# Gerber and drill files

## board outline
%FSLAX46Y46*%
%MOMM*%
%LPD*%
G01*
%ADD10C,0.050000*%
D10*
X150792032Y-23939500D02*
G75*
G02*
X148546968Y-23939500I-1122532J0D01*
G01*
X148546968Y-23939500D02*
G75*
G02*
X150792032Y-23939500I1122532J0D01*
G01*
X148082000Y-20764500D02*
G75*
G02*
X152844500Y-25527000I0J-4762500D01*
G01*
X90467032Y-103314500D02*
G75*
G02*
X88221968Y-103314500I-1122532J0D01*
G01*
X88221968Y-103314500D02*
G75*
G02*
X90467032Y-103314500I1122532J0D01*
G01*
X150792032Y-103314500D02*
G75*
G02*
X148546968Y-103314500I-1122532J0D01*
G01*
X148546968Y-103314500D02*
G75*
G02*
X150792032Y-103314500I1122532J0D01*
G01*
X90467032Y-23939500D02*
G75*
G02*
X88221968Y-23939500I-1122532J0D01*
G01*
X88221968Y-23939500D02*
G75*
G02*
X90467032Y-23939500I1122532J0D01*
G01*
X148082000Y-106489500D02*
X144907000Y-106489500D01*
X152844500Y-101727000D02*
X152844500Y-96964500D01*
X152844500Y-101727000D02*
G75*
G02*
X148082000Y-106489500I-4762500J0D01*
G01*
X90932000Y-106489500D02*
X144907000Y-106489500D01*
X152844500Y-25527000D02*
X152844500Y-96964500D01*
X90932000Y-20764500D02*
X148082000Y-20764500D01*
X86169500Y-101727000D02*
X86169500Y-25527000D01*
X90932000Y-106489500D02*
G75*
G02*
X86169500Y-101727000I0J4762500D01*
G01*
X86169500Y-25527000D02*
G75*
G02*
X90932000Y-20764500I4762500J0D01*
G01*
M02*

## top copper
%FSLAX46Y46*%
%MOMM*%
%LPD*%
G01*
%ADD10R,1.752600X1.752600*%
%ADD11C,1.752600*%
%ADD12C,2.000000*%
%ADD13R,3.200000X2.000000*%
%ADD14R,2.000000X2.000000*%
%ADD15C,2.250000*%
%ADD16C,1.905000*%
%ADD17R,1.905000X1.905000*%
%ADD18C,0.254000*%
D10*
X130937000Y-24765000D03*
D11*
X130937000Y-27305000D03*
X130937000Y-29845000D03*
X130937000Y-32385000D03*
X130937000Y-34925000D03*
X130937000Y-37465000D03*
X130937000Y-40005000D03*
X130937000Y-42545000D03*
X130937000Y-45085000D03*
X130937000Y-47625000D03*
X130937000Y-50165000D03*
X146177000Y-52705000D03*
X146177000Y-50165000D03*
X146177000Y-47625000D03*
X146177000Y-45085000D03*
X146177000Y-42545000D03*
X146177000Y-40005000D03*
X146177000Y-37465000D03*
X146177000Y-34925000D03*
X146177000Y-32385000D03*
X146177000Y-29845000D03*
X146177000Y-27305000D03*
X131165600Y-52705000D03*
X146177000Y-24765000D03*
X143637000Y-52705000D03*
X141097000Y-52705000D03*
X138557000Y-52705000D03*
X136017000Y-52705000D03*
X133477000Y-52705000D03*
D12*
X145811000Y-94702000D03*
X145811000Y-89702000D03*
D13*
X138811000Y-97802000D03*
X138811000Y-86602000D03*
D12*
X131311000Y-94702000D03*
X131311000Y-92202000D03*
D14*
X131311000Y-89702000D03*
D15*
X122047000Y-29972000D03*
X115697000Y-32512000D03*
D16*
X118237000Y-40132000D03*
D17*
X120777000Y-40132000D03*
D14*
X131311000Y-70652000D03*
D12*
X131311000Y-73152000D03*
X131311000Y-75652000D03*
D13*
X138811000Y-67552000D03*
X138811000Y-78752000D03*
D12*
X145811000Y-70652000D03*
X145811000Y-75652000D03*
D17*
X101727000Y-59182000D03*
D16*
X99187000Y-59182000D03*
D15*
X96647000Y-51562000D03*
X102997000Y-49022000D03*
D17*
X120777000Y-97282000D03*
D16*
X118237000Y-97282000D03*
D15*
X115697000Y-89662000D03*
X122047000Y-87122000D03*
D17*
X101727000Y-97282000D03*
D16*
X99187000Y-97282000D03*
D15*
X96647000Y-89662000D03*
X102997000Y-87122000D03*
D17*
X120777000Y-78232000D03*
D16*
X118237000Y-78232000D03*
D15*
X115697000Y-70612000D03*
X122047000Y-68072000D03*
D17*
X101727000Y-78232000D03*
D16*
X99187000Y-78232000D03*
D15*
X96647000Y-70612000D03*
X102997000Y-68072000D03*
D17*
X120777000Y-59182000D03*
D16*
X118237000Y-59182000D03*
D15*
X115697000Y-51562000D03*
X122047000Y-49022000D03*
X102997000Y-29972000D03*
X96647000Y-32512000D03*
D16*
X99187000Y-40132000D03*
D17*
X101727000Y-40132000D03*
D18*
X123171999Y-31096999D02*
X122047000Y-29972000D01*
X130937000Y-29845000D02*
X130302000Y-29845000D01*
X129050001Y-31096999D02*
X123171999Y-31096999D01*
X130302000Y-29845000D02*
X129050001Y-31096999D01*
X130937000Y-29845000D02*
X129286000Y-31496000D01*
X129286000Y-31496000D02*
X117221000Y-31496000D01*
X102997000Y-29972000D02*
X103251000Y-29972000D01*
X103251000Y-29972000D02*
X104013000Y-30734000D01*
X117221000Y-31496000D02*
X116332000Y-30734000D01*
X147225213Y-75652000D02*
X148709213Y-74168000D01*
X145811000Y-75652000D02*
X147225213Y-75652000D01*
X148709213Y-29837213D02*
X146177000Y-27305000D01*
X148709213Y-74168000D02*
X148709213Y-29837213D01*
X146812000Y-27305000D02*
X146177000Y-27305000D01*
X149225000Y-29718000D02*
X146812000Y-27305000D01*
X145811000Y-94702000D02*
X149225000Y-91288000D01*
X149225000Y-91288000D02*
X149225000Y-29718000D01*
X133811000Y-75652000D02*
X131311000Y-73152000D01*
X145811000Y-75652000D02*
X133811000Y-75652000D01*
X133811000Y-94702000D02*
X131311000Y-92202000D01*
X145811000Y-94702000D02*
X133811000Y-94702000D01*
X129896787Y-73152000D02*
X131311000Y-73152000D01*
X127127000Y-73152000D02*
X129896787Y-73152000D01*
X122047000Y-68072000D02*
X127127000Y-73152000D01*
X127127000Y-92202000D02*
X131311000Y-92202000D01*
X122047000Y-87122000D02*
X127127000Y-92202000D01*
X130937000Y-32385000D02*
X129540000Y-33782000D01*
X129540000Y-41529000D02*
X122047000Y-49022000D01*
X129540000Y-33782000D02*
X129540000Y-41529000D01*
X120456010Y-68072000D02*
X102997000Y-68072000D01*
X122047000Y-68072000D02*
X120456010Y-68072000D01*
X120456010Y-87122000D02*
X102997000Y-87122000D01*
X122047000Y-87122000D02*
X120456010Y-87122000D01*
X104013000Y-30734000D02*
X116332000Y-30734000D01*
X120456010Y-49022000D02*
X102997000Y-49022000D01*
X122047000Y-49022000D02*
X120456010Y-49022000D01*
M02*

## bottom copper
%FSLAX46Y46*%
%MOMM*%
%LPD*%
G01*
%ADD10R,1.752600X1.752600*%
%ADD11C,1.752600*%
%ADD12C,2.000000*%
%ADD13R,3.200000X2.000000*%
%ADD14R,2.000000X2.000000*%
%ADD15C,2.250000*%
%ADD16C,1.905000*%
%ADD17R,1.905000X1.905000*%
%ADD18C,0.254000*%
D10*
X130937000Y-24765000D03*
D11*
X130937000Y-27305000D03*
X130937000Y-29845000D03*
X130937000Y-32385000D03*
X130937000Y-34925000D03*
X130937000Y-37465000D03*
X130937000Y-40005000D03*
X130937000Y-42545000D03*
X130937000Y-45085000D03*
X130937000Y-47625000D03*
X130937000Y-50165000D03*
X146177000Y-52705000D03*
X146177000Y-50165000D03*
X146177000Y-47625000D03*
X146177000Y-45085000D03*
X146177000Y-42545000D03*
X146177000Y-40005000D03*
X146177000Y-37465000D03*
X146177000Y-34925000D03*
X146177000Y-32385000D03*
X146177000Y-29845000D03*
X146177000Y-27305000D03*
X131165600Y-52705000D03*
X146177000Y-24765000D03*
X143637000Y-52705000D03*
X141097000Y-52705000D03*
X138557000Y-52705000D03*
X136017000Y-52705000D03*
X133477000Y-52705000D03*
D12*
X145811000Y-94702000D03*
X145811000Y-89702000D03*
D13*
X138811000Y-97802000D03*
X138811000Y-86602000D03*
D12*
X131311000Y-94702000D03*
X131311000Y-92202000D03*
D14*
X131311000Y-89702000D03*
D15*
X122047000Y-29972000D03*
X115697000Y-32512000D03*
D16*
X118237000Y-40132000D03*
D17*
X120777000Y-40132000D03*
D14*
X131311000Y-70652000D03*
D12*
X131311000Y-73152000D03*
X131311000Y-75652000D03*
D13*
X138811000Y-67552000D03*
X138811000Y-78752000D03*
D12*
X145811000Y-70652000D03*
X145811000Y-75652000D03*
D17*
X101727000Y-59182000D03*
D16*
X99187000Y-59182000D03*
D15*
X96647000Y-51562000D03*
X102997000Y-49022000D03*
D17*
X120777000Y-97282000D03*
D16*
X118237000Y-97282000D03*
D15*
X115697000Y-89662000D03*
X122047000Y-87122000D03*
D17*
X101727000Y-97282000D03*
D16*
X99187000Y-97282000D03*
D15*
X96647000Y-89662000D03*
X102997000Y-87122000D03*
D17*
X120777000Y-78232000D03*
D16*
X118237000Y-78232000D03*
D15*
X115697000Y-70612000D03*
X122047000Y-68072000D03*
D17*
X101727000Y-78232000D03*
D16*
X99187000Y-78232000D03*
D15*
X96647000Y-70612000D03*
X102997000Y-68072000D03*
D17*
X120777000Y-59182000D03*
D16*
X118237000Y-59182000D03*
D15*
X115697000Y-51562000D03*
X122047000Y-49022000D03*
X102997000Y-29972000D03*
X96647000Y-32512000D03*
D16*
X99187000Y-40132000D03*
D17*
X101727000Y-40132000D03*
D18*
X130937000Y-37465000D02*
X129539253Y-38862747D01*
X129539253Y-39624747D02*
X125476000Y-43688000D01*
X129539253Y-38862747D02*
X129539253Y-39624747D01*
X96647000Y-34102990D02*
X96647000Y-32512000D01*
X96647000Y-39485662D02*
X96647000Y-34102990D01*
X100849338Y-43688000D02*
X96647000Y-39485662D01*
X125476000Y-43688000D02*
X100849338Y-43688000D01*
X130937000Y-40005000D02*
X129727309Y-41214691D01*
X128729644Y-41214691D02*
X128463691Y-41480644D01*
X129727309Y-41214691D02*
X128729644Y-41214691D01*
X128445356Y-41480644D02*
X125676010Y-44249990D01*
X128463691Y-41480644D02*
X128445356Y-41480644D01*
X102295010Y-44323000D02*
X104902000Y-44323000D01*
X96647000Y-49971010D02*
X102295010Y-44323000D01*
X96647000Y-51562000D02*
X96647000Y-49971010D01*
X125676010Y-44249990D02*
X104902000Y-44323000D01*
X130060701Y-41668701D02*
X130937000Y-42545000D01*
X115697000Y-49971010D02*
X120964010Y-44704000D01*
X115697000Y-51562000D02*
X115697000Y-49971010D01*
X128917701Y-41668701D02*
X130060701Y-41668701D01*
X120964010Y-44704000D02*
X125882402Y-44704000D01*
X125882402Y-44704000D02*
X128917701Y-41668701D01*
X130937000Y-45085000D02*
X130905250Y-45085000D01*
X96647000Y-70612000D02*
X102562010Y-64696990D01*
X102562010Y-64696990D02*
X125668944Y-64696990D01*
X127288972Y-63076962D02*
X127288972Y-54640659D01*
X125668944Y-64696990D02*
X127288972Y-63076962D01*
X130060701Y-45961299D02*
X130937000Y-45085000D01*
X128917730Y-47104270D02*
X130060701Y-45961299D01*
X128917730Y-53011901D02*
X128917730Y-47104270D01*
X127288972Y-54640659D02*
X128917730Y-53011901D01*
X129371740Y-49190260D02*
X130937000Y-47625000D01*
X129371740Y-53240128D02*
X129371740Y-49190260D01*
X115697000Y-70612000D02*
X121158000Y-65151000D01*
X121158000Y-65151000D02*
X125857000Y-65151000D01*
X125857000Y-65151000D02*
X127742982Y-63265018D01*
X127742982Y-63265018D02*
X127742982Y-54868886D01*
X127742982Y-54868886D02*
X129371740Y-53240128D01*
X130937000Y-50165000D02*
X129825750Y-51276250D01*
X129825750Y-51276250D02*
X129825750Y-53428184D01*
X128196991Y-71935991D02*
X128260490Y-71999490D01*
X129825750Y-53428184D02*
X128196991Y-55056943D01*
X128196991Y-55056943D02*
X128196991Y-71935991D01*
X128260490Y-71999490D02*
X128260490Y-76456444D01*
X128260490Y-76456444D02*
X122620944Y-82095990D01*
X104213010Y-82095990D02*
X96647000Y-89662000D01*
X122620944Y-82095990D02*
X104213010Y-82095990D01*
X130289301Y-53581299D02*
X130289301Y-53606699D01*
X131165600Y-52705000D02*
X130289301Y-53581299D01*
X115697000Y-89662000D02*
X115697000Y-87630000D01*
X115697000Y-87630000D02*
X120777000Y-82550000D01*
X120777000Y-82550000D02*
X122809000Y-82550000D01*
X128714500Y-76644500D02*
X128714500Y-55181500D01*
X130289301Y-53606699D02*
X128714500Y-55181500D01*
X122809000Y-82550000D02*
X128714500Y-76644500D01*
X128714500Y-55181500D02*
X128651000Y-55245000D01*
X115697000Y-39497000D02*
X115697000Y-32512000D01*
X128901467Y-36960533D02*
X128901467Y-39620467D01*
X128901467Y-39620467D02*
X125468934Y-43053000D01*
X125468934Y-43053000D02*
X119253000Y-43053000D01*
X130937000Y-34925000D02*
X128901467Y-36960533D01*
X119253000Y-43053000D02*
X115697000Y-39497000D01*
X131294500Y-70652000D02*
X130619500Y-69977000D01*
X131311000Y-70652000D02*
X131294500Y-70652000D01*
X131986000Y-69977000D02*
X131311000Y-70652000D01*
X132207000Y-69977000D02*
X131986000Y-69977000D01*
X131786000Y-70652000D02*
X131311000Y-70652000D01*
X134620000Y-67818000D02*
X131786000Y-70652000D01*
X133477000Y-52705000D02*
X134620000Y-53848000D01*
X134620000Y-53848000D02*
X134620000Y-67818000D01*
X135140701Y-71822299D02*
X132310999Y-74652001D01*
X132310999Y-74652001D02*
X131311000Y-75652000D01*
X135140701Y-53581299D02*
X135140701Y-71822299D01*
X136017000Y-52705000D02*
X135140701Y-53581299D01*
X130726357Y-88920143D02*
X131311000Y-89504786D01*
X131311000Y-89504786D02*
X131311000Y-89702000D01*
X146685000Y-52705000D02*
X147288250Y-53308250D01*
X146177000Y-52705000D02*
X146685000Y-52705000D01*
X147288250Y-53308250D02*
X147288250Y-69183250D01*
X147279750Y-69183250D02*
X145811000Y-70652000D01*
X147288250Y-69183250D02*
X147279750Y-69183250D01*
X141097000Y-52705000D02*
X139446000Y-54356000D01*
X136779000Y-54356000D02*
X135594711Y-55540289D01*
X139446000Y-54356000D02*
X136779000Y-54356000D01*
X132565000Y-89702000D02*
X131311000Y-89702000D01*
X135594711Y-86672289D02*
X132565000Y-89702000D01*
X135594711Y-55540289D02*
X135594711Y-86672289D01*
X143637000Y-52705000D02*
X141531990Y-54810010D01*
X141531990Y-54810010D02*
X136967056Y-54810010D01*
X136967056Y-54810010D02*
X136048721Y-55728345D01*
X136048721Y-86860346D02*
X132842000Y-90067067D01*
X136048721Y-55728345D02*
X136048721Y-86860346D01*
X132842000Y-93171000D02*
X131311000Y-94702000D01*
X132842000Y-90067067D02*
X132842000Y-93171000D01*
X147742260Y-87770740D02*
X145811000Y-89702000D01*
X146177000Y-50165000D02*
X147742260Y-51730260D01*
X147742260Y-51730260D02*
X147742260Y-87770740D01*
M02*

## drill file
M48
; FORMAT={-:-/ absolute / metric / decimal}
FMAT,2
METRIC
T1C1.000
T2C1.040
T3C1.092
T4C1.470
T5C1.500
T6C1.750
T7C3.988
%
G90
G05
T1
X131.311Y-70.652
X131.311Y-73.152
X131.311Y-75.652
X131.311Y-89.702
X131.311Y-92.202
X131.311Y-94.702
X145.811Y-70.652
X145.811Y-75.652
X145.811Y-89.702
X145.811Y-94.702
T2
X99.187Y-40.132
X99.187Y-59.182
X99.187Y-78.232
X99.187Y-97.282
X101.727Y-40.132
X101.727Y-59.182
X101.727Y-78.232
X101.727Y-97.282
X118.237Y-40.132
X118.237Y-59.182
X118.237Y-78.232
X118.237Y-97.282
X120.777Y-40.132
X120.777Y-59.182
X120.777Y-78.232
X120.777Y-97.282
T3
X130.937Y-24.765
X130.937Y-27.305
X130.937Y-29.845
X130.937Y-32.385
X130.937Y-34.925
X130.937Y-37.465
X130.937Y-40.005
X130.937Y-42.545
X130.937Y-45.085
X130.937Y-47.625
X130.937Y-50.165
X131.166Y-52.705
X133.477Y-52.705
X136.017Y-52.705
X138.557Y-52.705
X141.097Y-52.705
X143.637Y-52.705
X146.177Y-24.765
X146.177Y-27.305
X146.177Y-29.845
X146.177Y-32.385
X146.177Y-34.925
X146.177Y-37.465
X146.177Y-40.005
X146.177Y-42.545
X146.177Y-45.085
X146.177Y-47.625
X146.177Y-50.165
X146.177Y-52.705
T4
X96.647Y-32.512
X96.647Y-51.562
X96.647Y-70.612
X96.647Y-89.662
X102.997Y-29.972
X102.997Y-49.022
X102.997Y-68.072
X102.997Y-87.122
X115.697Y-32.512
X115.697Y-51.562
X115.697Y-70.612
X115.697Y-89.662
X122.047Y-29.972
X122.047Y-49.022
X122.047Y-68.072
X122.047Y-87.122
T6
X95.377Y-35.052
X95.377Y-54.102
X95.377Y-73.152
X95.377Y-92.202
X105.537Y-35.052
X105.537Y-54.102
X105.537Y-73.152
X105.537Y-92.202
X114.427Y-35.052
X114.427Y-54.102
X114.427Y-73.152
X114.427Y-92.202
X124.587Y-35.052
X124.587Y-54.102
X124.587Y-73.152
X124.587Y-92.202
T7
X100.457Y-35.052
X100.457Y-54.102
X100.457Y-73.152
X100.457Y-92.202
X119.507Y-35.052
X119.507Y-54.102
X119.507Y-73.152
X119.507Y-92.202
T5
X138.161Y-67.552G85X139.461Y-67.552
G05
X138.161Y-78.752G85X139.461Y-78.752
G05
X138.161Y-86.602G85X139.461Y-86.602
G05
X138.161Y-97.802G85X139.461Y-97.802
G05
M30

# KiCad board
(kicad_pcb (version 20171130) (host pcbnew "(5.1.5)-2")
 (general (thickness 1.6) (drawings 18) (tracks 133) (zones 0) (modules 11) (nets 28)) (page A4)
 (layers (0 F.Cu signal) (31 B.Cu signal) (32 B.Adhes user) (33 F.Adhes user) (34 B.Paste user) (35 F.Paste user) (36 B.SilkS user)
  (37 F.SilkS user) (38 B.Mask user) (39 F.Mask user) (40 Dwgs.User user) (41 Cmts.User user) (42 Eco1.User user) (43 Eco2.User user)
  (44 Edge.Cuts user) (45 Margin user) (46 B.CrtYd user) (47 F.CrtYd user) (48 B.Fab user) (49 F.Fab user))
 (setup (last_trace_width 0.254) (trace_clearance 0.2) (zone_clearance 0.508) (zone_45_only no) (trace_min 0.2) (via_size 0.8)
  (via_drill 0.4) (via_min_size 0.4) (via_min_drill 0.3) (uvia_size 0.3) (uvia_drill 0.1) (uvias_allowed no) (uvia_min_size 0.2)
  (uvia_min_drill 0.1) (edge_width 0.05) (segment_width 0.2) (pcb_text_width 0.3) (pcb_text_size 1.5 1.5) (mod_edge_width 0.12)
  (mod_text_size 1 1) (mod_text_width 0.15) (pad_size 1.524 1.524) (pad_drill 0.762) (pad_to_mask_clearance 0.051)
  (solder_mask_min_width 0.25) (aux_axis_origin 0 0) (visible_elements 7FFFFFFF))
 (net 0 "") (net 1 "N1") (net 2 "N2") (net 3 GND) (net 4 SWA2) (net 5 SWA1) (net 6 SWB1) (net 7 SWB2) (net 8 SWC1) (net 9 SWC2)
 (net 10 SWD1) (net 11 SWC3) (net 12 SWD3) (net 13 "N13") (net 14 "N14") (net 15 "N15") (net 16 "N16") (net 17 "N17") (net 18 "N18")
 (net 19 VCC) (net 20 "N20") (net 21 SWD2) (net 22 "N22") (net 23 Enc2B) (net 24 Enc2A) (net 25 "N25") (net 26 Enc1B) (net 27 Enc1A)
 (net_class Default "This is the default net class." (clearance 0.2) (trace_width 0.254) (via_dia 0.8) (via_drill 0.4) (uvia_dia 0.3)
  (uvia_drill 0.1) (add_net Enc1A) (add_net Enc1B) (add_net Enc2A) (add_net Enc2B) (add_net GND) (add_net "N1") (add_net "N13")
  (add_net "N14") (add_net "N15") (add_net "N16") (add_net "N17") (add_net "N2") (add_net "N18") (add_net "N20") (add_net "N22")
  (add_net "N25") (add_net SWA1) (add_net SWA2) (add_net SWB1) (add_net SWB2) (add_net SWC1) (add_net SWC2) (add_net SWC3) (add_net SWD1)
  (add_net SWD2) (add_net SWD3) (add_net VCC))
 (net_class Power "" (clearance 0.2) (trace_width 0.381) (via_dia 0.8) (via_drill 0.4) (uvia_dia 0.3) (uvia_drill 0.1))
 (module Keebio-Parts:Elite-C (layer F.Cu) (at 138.557 38.735 270)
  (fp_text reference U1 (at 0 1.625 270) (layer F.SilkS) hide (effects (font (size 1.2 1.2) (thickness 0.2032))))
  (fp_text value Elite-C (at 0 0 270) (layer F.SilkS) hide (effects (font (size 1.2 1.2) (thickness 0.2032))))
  (pad 1 thru_hole rect (at -13.97 7.62 270) (size 1.7526 1.7526) (drill 1.0922) (layers *.Cu *.SilkS *.Mask) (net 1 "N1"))
  (pad 2 thru_hole circle (at -11.43 7.62 270) (size 1.7526 1.7526) (drill 1.0922) (layers *.Cu *.SilkS *.Mask) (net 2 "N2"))
  (pad 3 thru_hole circle (at -8.89 7.62 270) (size 1.7526 1.7526) (drill 1.0922) (layers *.Cu *.SilkS *.Mask) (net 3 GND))
  (pad 4 thru_hole circle (at -6.35 7.62 270) (size 1.7526 1.7526) (drill 1.0922) (layers *.Cu *.SilkS *.Mask) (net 3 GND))
  (pad 5 thru_hole circle (at -3.81 7.62 270) (size 1.7526 1.7526) (drill 1.0922) (layers *.Cu *.SilkS *.Mask) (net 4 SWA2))
  (pad 6 thru_hole circle (at -1.27 7.62 270) (size 1.7526 1.7526) (drill 1.0922) (layers *.Cu *.SilkS *.Mask) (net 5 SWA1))
  (pad 7 thru_hole circle (at 1.27 7.62 270) (size 1.7526 1.7526) (drill 1.0922) (layers *.Cu *.SilkS *.Mask) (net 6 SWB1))
  (pad 8 thru_hole circle (at 3.81 7.62 270) (size 1.7526 1.7526) (drill 1.0922) (layers *.Cu *.SilkS *.Mask) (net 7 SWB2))
  (pad 9 thru_hole circle (at 6.35 7.62 270) (size 1.7526 1.7526) (drill 1.0922) (layers *.Cu *.SilkS *.Mask) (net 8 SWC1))
  (pad 10 thru_hole circle (at 8.89 7.62 270) (size 1.7526 1.7526) (drill 1.0922) (layers *.Cu *.SilkS *.Mask) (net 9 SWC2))
  (pad 11 thru_hole circle (at 11.43 7.62 270) (size 1.7526 1.7526) (drill 1.0922) (layers *.Cu *.SilkS *.Mask) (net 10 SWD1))
  (pad 13 thru_hole circle (at 13.97 -7.62 270) (size 1.7526 1.7526) (drill 1.0922) (layers *.Cu *.SilkS *.Mask) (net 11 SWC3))
  (pad 14 thru_hole circle (at 11.43 -7.62 270) (size 1.7526 1.7526) (drill 1.0922) (layers *.Cu *.SilkS *.Mask) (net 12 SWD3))
  (pad 15 thru_hole circle (at 8.89 -7.62 270) (size 1.7526 1.7526) (drill 1.0922) (layers *.Cu *.SilkS *.Mask) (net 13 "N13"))
  (pad 16 thru_hole circle (at 6.35 -7.62 270) (size 1.7526 1.7526) (drill 1.0922) (layers *.Cu *.SilkS *.Mask) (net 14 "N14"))
  (pad 17 thru_hole circle (at 3.81 -7.62 270) (size 1.7526 1.7526) (drill 1.0922) (layers *.Cu *.SilkS *.Mask) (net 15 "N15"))
  (pad 18 thru_hole circle (at 1.27 -7.62 270) (size 1.7526 1.7526) (drill 1.0922) (layers *.Cu *.SilkS *.Mask) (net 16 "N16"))
  (pad 19 thru_hole circle (at -1.27 -7.62 270) (size 1.7526 1.7526) (drill 1.0922) (layers *.Cu *.SilkS *.Mask) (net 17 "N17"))
  (pad 20 thru_hole circle (at -3.81 -7.62 270) (size 1.7526 1.7526) (drill 1.0922) (layers *.Cu *.SilkS *.Mask) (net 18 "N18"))
  (pad 21 thru_hole circle (at -6.35 -7.62 270) (size 1.7526 1.7526) (drill 1.0922) (layers *.Cu *.SilkS *.Mask) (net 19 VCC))
  (pad 22 thru_hole circle (at -8.89 -7.62 270) (size 1.7526 1.7526) (drill 1.0922) (layers *.Cu *.SilkS *.Mask) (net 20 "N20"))
  (pad 23 thru_hole circle (at -11.43 -7.62 270) (size 1.7526 1.7526) (drill 1.0922) (layers *.Cu *.SilkS *.Mask) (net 3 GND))
  (pad 12 thru_hole circle (at 13.97 7.3914 270) (size 1.7526 1.7526) (drill 1.0922) (layers *.Cu *.SilkS *.Mask) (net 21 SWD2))
  (pad 24 thru_hole circle (at -13.97 -7.62 270) (size 1.7526 1.7526) (drill 1.0922) (layers *.Cu *.SilkS *.Mask) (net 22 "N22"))
  (pad 29 thru_hole circle (at 13.97 -5.08 270) (size 1.7526 1.7526) (drill 1.0922) (layers *.Cu *.SilkS *.Mask) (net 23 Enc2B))
  (pad 28 thru_hole circle (at 13.97 -2.54 270) (size 1.7526 1.7526) (drill 1.0922) (layers *.Cu *.SilkS *.Mask) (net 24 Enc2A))
  (pad 27 thru_hole circle (at 13.97 0 270) (size 1.7526 1.7526) (drill 1.0922) (layers *.Cu *.SilkS *.Mask) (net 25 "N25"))
  (pad 26 thru_hole circle (at 13.97 2.54 270) (size 1.7526 1.7526) (drill 1.0922) (layers *.Cu *.SilkS *.Mask) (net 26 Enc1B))
  (pad 25 thru_hole circle (at 13.97 5.08 270) (size 1.7526 1.7526) (drill 1.0922) (layers *.Cu *.SilkS *.Mask) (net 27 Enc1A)))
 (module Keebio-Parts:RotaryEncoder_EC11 (layer F.Cu) (at 138.811 92.202)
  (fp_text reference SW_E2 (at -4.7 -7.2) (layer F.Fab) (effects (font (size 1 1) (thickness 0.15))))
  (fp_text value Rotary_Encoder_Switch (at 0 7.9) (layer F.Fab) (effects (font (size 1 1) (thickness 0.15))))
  (pad S1 thru_hole circle (at 7 2.5) (size 2 2) (drill 1) (layers *.Cu *.Mask) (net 3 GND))
  (pad S2 thru_hole circle (at 7 -2.5) (size 2 2) (drill 1) (layers *.Cu *.Mask) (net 12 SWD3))
  (pad "" np_thru_hole rect (at 0 5.6) (size 3.2 2) (drill oval 2.8 1.5) (layers *.Cu *.Mask))
  (pad "" np_thru_hole rect (at 0 -5.6) (size 3.2 2) (drill oval 2.8 1.5) (layers *.Cu *.Mask))
  (pad B thru_hole circle (at -7.5 2.5) (size 2 2) (drill 1) (layers *.Cu *.Mask) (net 23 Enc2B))
  (pad C thru_hole circle (at -7.5 0) (size 2 2) (drill 1) (layers *.Cu *.Mask) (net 3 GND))
  (pad A thru_hole rect (at -7.5 -2.5) (size 2 2) (drill 1) (layers *.Cu *.Mask) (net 24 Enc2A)))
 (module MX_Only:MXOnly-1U (layer F.Cu) (at 119.507 35.052)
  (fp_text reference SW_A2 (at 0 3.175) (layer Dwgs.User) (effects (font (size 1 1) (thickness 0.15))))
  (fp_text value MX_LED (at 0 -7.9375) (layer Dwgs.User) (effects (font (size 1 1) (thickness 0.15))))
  (pad 2 thru_hole circle (at 2.54 -5.08) (size 2.25 2.25) (drill 1.47) (layers *.Cu B.Mask) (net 3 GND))
  (pad "" np_thru_hole circle (at 0 0) (size 3.9878 3.9878) (drill 3.9878) (layers *.Cu *.Mask))
  (pad 1 thru_hole circle (at -3.81 -2.54) (size 2.25 2.25) (drill 1.47) (layers *.Cu B.Mask) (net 4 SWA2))
  (pad 3 thru_hole circle (at -1.27 5.08) (size 1.905 1.905) (drill 1.04) (layers *.Cu B.Mask))
  (pad 4 thru_hole rect (at 1.27 5.08) (size 1.905 1.905) (drill 1.04) (layers *.Cu B.Mask))
  (pad "" np_thru_hole circle (at -5.08 0 48.0996) (size 1.75 1.75) (drill 1.75) (layers *.Cu *.Mask))
  (pad "" np_thru_hole circle (at 5.08 0 48.0996) (size 1.75 1.75) (drill 1.75) (layers *.Cu *.Mask)))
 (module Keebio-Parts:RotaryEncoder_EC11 (layer F.Cu) (at 138.811 73.152)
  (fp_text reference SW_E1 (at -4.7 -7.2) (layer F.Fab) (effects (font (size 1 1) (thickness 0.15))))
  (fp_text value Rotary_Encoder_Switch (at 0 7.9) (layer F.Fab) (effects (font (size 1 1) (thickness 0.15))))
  (pad A thru_hole rect (at -7.5 -2.5) (size 2 2) (drill 1) (layers *.Cu *.Mask) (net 27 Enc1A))
  (pad C thru_hole circle (at -7.5 0) (size 2 2) (drill 1) (layers *.Cu *.Mask) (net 3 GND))
  (pad B thru_hole circle (at -7.5 2.5) (size 2 2) (drill 1) (layers *.Cu *.Mask) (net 26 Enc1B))
  (pad "" np_thru_hole rect (at 0 -5.6) (size 3.2 2) (drill oval 2.8 1.5) (layers *.Cu *.Mask))
  (pad "" np_thru_hole rect (at 0 5.6) (size 3.2 2) (drill oval 2.8 1.5) (layers *.Cu *.Mask))
  (pad S2 thru_hole circle (at 7 -2.5) (size 2 2) (drill 1) (layers *.Cu *.Mask) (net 11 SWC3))
  (pad S1 thru_hole circle (at 7 2.5) (size 2 2) (drill 1) (layers *.Cu *.Mask) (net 3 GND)))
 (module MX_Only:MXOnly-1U (layer F.Cu) (at 100.457 54.102)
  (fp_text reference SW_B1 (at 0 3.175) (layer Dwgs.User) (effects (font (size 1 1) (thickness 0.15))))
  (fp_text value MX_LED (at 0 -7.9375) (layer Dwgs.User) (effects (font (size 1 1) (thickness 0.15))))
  (pad "" np_thru_hole circle (at 5.08 0 48.0996) (size 1.75 1.75) (drill 1.75) (layers *.Cu *.Mask))
  (pad "" np_thru_hole circle (at -5.08 0 48.0996) (size 1.75 1.75) (drill 1.75) (layers *.Cu *.Mask))
  (pad 4 thru_hole rect (at 1.27 5.08) (size 1.905 1.905) (drill 1.04) (layers *.Cu B.Mask))
  (pad 3 thru_hole circle (at -1.27 5.08) (size 1.905 1.905) (drill 1.04) (layers *.Cu B.Mask))
  (pad 1 thru_hole circle (at -3.81 -2.54) (size 2.25 2.25) (drill 1.47) (layers *.Cu B.Mask) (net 6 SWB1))
  (pad "" np_thru_hole circle (at 0 0) (size 3.9878 3.9878) (drill 3.9878) (layers *.Cu *.Mask))
  (pad 2 thru_hole circle (at 2.54 -5.08) (size 2.25 2.25) (drill 1.47) (layers *.Cu B.Mask) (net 3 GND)))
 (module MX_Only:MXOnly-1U (layer F.Cu) (at 119.507 92.202)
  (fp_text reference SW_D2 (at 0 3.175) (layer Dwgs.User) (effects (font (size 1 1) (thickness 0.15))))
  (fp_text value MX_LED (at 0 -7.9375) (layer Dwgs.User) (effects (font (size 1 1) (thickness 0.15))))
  (pad "" np_thru_hole circle (at 5.08 0 48.0996) (size 1.75 1.75) (drill 1.75) (layers *.Cu *.Mask))
  (pad "" np_thru_hole circle (at -5.08 0 48.0996) (size 1.75 1.75) (drill 1.75) (layers *.Cu *.Mask))
  (pad 4 thru_hole rect (at 1.27 5.08) (size 1.905 1.905) (drill 1.04) (layers *.Cu B.Mask))
  (pad 3 thru_hole circle (at -1.27 5.08) (size 1.905 1.905) (drill 1.04) (layers *.Cu B.Mask))
  (pad 1 thru_hole circle (at -3.81 -2.54) (size 2.25 2.25) (drill 1.47) (layers *.Cu B.Mask) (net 21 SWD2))
  (pad "" np_thru_hole circle (at 0 0) (size 3.9878 3.9878) (drill 3.9878) (layers *.Cu *.Mask))
  (pad 2 thru_hole circle (at 2.54 -5.08) (size 2.25 2.25) (drill 1.47) (layers *.Cu B.Mask) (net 3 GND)))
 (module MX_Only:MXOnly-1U (layer F.Cu) (at 100.457 92.202)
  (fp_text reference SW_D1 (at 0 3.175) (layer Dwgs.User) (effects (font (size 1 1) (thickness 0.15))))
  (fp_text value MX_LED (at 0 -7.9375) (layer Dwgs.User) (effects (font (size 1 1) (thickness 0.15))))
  (pad "" np_thru_hole circle (at 5.08 0 48.0996) (size 1.75 1.75) (drill 1.75) (layers *.Cu *.Mask))
  (pad "" np_thru_hole circle (at -5.08 0 48.0996) (size 1.75 1.75) (drill 1.75) (layers *.Cu *.Mask))
  (pad 4 thru_hole rect (at 1.27 5.08) (size 1.905 1.905) (drill 1.04) (layers *.Cu B.Mask))
  (pad 3 thru_hole circle (at -1.27 5.08) (size 1.905 1.905) (drill 1.04) (layers *.Cu B.Mask))
  (pad 1 thru_hole circle (at -3.81 -2.54) (size 2.25 2.25) (drill 1.47) (layers *.Cu B.Mask) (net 10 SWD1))
  (pad "" np_thru_hole circle (at 0 0) (size 3.9878 3.9878) (drill 3.9878) (layers *.Cu *.Mask))
  (pad 2 thru_hole circle (at 2.54 -5.08) (size 2.25 2.25) (drill 1.47) (layers *.Cu B.Mask) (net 3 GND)))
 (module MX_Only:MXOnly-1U (layer F.Cu) (at 119.507 73.152)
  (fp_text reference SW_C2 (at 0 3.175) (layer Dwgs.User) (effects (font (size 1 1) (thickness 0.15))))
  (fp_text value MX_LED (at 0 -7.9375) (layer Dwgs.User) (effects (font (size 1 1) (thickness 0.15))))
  (pad "" np_thru_hole circle (at 5.08 0 48.0996) (size 1.75 1.75) (drill 1.75) (layers *.Cu *.Mask))
  (pad "" np_thru_hole circle (at -5.08 0 48.0996) (size 1.75 1.75) (drill 1.75) (layers *.Cu *.Mask))
  (pad 4 thru_hole rect (at 1.27 5.08) (size 1.905 1.905) (drill 1.04) (layers *.Cu B.Mask))
  (pad 3 thru_hole circle (at -1.27 5.08) (size 1.905 1.905) (drill 1.04) (layers *.Cu B.Mask))
  (pad 1 thru_hole circle (at -3.81 -2.54) (size 2.25 2.25) (drill 1.47) (layers *.Cu B.Mask) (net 9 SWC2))
  (pad "" np_thru_hole circle (at 0 0) (size 3.9878 3.9878) (drill 3.9878) (layers *.Cu *.Mask))
  (pad 2 thru_hole circle (at 2.54 -5.08) (size 2.25 2.25) (drill 1.47) (layers *.Cu B.Mask) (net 3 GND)))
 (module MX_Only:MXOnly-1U (layer F.Cu) (at 100.457 73.152)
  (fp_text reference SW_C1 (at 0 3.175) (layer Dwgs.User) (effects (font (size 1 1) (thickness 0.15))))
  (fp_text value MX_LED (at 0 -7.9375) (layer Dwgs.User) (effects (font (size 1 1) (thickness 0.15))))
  (pad "" np_thru_hole circle (at 5.08 0 48.0996) (size 1.75 1.75) (drill 1.75) (layers *.Cu *.Mask))
  (pad "" np_thru_hole circle (at -5.08 0 48.0996) (size 1.75 1.75) (drill 1.75) (layers *.Cu *.Mask))
  (pad 4 thru_hole rect (at 1.27 5.08) (size 1.905 1.905) (drill 1.04) (layers *.Cu B.Mask))
  (pad 3 thru_hole circle (at -1.27 5.08) (size 1.905 1.905) (drill 1.04) (layers *.Cu B.Mask))
  (pad 1 thru_hole circle (at -3.81 -2.54) (size 2.25 2.25) (drill 1.47) (layers *.Cu B.Mask) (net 8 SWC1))
  (pad "" np_thru_hole circle (at 0 0) (size 3.9878 3.9878) (drill 3.9878) (layers *.Cu *.Mask))
  (pad 2 thru_hole circle (at 2.54 -5.08) (size 2.25 2.25) (drill 1.47) (layers *.Cu B.Mask) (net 3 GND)))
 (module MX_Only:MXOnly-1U (layer F.Cu) (at 119.507 54.102)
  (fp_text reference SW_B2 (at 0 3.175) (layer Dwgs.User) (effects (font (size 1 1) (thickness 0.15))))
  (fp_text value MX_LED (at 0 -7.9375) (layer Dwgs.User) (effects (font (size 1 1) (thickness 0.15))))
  (pad "" np_thru_hole circle (at 5.08 0 48.0996) (size 1.75 1.75) (drill 1.75) (layers *.Cu *.Mask))
  (pad "" np_thru_hole circle (at -5.08 0 48.0996) (size 1.75 1.75) (drill 1.75) (layers *.Cu *.Mask))
  (pad 4 thru_hole rect (at 1.27 5.08) (size 1.905 1.905) (drill 1.04) (layers *.Cu B.Mask))
  (pad 3 thru_hole circle (at -1.27 5.08) (size 1.905 1.905) (drill 1.04) (layers *.Cu B.Mask))
  (pad 1 thru_hole circle (at -3.81 -2.54) (size 2.25 2.25) (drill 1.47) (layers *.Cu B.Mask) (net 7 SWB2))
  (pad "" np_thru_hole circle (at 0 0) (size 3.9878 3.9878) (drill 3.9878) (layers *.Cu *.Mask))
  (pad 2 thru_hole circle (at 2.54 -5.08) (size 2.25 2.25) (drill 1.47) (layers *.Cu B.Mask) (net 3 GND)))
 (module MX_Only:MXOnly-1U (layer F.Cu) (at 100.457 35.052)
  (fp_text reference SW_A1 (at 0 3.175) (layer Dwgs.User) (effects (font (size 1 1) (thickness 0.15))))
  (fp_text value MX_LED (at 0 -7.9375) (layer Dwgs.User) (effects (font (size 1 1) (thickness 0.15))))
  (pad 2 thru_hole circle (at 2.54 -5.08) (size 2.25 2.25) (drill 1.47) (layers *.Cu B.Mask) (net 3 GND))
  (pad "" np_thru_hole circle (at 0 0) (size 3.9878 3.9878) (drill 3.9878) (layers *.Cu *.Mask))
  (pad 1 thru_hole circle (at -3.81 -2.54) (size 2.25 2.25) (drill 1.47) (layers *.Cu B.Mask) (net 5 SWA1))
  (pad 3 thru_hole circle (at -1.27 5.08) (size 1.905 1.905) (drill 1.04) (layers *.Cu B.Mask))
  (pad 4 thru_hole rect (at 1.27 5.08) (size 1.905 1.905) (drill 1.04) (layers *.Cu B.Mask))
  (pad "" np_thru_hole circle (at -5.08 0 48.0996) (size 1.75 1.75) (drill 1.75) (layers *.Cu *.Mask))
  (pad "" np_thru_hole circle (at 5.08 0 48.0996) (size 1.75 1.75) (drill 1.75) (layers *.Cu *.Mask)))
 (gr_circle (center 149.6695 23.9395) (end 150.46325 24.73325) (layer Edge.Cuts) (width 0.05))
 (gr_arc (start 148.082 25.527) (end 152.8445 25.527) (angle -90) (layer Edge.Cuts) (width 0.05))
 (gr_circle (center 89.3445 103.3145) (end 90.13825 104.10825) (layer Edge.Cuts) (width 0.05))
 (gr_circle (center 149.6695 103.3145) (end 150.46325 104.10825) (layer Edge.Cuts) (width 0.05))
 (gr_circle (center 89.3445 23.9395) (end 90.13825 24.73325) (layer Edge.Cuts) (width 0.05))
 (gr_line (start 148.082 106.4895) (end 144.907 106.4895) (layer Edge.Cuts) (width 0.05))
 (gr_line (start 152.8445 101.727) (end 152.8445 96.9645) (layer Edge.Cuts) (width 0.05))
 (gr_arc (start 148.082 101.727) (end 148.082 106.4895) (angle -90) (layer Edge.Cuts) (width 0.05))
 (gr_line (start 90.932 106.4895) (end 144.907 106.4895) (layer Edge.Cuts) (width 0.05))
 (gr_line (start 152.8445 25.527) (end 152.8445 96.9645) (layer Edge.Cuts) (width 0.05))
 (gr_line (start 90.932 20.7645) (end 148.082 20.7645) (layer Edge.Cuts) (width 0.05))
 (gr_line (start 86.1695 101.727) (end 86.1695 25.527) (layer Edge.Cuts) (width 0.05))
 (gr_arc (start 90.932 101.727) (end 86.1695 101.727) (angle -90) (layer Edge.Cuts) (width 0.05))
 (gr_arc (start 90.932 25.527) (end 90.932 20.7645) (angle -90) (layer Edge.Cuts) (width 0.05))
 (segment (start 123.171999 31.096999) (end 122.047 29.972) (width 0.254) (layer F.Cu) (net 3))
 (segment (start 130.937 29.845) (end 130.302 29.845) (width 0.254) (layer F.Cu) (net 3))
 (segment (start 129.050001 31.096999) (end 123.171999 31.096999) (width 0.254) (layer F.Cu) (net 3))
 (segment (start 130.302 29.845) (end 129.050001 31.096999) (width 0.254) (layer F.Cu) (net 3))
 (segment (start 130.937 29.845) (end 129.286 31.496) (width 0.254) (layer F.Cu) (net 3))
 (segment (start 129.286 31.496) (end 117.221 31.496) (width 0.254) (layer F.Cu) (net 3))
 (segment (start 102.997 29.972) (end 103.251 29.972) (width 0.254) (layer F.Cu) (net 3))
 (segment (start 103.251 29.972) (end 104.013 30.734) (width 0.254) (layer F.Cu) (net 3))
 (segment (start 117.221 31.496) (end 116.332 30.734) (width 0.254) (layer F.Cu) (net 3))
 (segment (start 147.225213 75.652) (end 148.709213 74.168) (width 0.254) (layer F.Cu) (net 3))
 (segment (start 145.811 75.652) (end 147.225213 75.652) (width 0.254) (layer F.Cu) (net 3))
 (segment (start 148.709213 29.837213) (end 146.177 27.305) (width 0.254) (layer F.Cu) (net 3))
 (segment (start 148.709213 74.168) (end 148.709213 29.837213) (width 0.254) (layer F.Cu) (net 3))
 (segment (start 146.812 27.305) (end 146.177 27.305) (width 0.254) (layer F.Cu) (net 3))
 (segment (start 149.225 29.718) (end 146.812 27.305) (width 0.254) (layer F.Cu) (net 3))
 (segment (start 145.811 94.702) (end 149.225 91.288) (width 0.254) (layer F.Cu) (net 3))
 (segment (start 149.225 91.288) (end 149.225 29.718) (width 0.254) (layer F.Cu) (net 3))
 (segment (start 133.811 75.652) (end 131.311 73.152) (width 0.254) (layer F.Cu) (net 3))
 (segment (start 145.811 75.652) (end 133.811 75.652) (width 0.254) (layer F.Cu) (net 3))
 (segment (start 133.811 94.702) (end 131.311 92.202) (width 0.254) (layer F.Cu) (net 3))
 (segment (start 145.811 94.702) (end 133.811 94.702) (width 0.254) (layer F.Cu) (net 3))
 (segment (start 129.896787 73.152) (end 131.311 73.152) (width 0.254) (layer F.Cu) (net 3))
 (segment (start 127.127 73.152) (end 129.896787 73.152) (width 0.254) (layer F.Cu) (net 3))
 (segment (start 122.047 68.072) (end 127.127 73.152) (width 0.254) (layer F.Cu) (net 3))
 (segment (start 127.127 92.202) (end 131.311 92.202) (width 0.254) (layer F.Cu) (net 3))
 (segment (start 122.047 87.122) (end 127.127 92.202) (width 0.254) (layer F.Cu) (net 3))
 (segment (start 130.937 32.385) (end 129.54 33.782) (width 0.254) (layer F.Cu) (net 3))
 (segment (start 129.54 41.529) (end 122.047 49.022) (width 0.254) (layer F.Cu) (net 3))
 (segment (start 129.54 33.782) (end 129.54 41.529) (width 0.254) (layer F.Cu) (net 3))
 (segment (start 120.45601 68.072) (end 102.997 68.072) (width 0.254) (layer F.Cu) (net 3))
 (segment (start 122.047 68.072) (end 120.45601 68.072) (width 0.254) (layer F.Cu) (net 3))
 (segment (start 120.45601 87.122) (end 102.997 87.122) (width 0.254) (layer F.Cu) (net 3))
 (segment (start 122.047 87.122) (end 120.45601 87.122) (width 0.254) (layer F.Cu) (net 3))
 (segment (start 130.937 37.465) (end 129.539253 38.862747) (width 0.254) (layer B.Cu) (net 5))
 (segment (start 129.539253 39.624747) (end 125.476 43.688) (width 0.254) (layer B.Cu) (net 5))
 (segment (start 129.539253 38.862747) (end 129.539253 39.624747) (width 0.254) (layer B.Cu) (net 5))
 (segment (start 96.647 34.10299) (end 96.647 32.512) (width 0.254) (layer B.Cu) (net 5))
 (segment (start 96.647 39.485662) (end 96.647 34.10299) (width 0.254) (layer B.Cu) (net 5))
 (segment (start 100.849338 43.688) (end 96.647 39.485662) (width 0.254) (layer B.Cu) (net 5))
 (segment (start 125.476 43.688) (end 100.849338 43.688) (width 0.254) (layer B.Cu) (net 5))
 (segment (start 104.013 30.734) (end 116.332 30.734) (width 0.254) (layer F.Cu) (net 3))
 (segment (start 120.45601 49.022) (end 102.997 49.022) (width 0.254) (layer F.Cu) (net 3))
 (segment (start 122.047 49.022) (end 120.45601 49.022) (width 0.254) (layer F.Cu) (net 3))
 (segment (start 130.937 40.005) (end 129.727309 41.214691) (width 0.254) (layer B.Cu) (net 6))
 (segment (start 128.729644 41.214691) (end 128.463691 41.480644) (width 0.254) (layer B.Cu) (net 6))
 (segment (start 129.727309 41.214691) (end 128.729644 41.214691) (width 0.254) (layer B.Cu) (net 6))
 (segment (start 128.445356 41.480644) (end 125.67601 44.24999) (width 0.254) (layer B.Cu) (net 6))
 (segment (start 128.463691 41.480644) (end 128.445356 41.480644) (width 0.254) (layer B.Cu) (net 6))
 (segment (start 102.29501 44.323) (end 104.902 44.323) (width 0.254) (layer B.Cu) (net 6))
 (segment (start 96.647 49.97101) (end 102.29501 44.323) (width 0.254) (layer B.Cu) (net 6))
 (segment (start 96.647 51.562) (end 96.647 49.97101) (width 0.254) (layer B.Cu) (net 6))
 (segment (start 125.67601 44.24999) (end 104.902 44.323) (width 0.254) (layer B.Cu) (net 6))
 (segment (start 130.060701 41.668701) (end 130.937 42.545) (width 0.254) (layer B.Cu) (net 7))
 (segment (start 115.697 49.97101) (end 120.96401 44.704) (width 0.254) (layer B.Cu) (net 7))
 (segment (start 115.697 51.562) (end 115.697 49.97101) (width 0.254) (layer B.Cu) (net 7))
 (segment (start 128.917701 41.668701) (end 130.060701 41.668701) (width 0.254) (layer B.Cu) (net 7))
 (segment (start 120.96401 44.704) (end 125.882402 44.704) (width 0.254) (layer B.Cu) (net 7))
 (segment (start 125.882402 44.704) (end 128.917701 41.668701) (width 0.254) (layer B.Cu) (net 7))
 (segment (start 130.937 45.085) (end 130.90525 45.085) (width 0.254) (layer B.Cu) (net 8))
 (segment (start 96.647 70.612) (end 102.56201 64.69699) (width 0.254) (layer B.Cu) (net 8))
 (segment (start 102.56201 64.69699) (end 125.668944 64.69699) (width 0.254) (layer B.Cu) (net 8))
 (segment (start 127.288972 63.076962) (end 127.288972 54.640659) (width 0.254) (layer B.Cu) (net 8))
 (segment (start 125.668944 64.69699) (end 127.288972 63.076962) (width 0.254) (layer B.Cu) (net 8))
 (segment (start 130.060701 45.961299) (end 130.937 45.085) (width 0.254) (layer B.Cu) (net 8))
 (segment (start 128.91773 47.10427) (end 130.060701 45.961299) (width 0.254) (layer B.Cu) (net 8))
 (segment (start 128.91773 53.011901) (end 128.91773 47.10427) (width 0.254) (layer B.Cu) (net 8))
 (segment (start 127.288972 54.640659) (end 128.91773 53.011901) (width 0.254) (layer B.Cu) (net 8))
 (segment (start 129.37174 49.19026) (end 130.937 47.625) (width 0.254) (layer B.Cu) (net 9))
 (segment (start 129.37174 53.240128) (end 129.37174 49.19026) (width 0.254) (layer B.Cu) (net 9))
 (segment (start 115.697 70.612) (end 121.158 65.151) (width 0.254) (layer B.Cu) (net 9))
 (segment (start 121.158 65.151) (end 125.857 65.151) (width 0.254) (layer B.Cu) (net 9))
 (segment (start 125.857 65.151) (end 127.742982 63.265018) (width 0.254) (layer B.Cu) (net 9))
 (segment (start 127.742982 63.265018) (end 127.742982 54.868886) (width 0.254) (layer B.Cu) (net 9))
 (segment (start 127.742982 54.868886) (end 129.37174 53.240128) (width 0.254) (layer B.Cu) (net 9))
 (segment (start 130.937 50.165) (end 129.82575 51.27625) (width 0.254) (layer B.Cu) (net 10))
 (segment (start 129.82575 51.27625) (end 129.82575 53.428184) (width 0.254) (layer B.Cu) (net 10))
 (segment (start 128.196991 71.935991) (end 128.26049 71.99949) (width 0.254) (layer B.Cu) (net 10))
 (segment (start 129.82575 53.428184) (end 128.196991 55.056943) (width 0.254) (layer B.Cu) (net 10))
 (segment (start 128.196991 55.056943) (end 128.196991 71.935991) (width 0.254) (layer B.Cu) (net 10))
 (segment (start 128.26049 71.99949) (end 128.26049 76.456444) (width 0.254) (layer B.Cu) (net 10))
 (segment (start 128.26049 76.456444) (end 122.620944 82.09599) (width 0.254) (layer B.Cu) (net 10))
 (segment (start 104.21301 82.09599) (end 96.647 89.662) (width 0.254) (layer B.Cu) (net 10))
 (segment (start 122.620944 82.09599) (end 104.21301 82.09599) (width 0.254) (layer B.Cu) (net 10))
 (segment (start 130.289301 53.581299) (end 130.289301 53.606699) (width 0.254) (layer B.Cu) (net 21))
 (segment (start 131.1656 52.705) (end 130.289301 53.581299) (width 0.254) (layer B.Cu) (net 21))
 (segment (start 115.697 89.662) (end 115.697 87.63) (width 0.254) (layer B.Cu) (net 21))
 (segment (start 115.697 87.63) (end 120.777 82.55) (width 0.254) (layer B.Cu) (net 21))
 (segment (start 120.777 82.55) (end 122.809 82.55) (width 0.254) (layer B.Cu) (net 21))
 (segment (start 128.7145 76.6445) (end 128.7145 55.1815) (width 0.254) (layer B.Cu) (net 21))
 (segment (start 130.289301 53.606699) (end 128.7145 55.1815) (width 0.254) (layer B.Cu) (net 21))
 (segment (start 122.809 82.55) (end 128.7145 76.6445) (width 0.254) (layer B.Cu) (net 21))
 (segment (start 128.7145 55.1815) (end 128.651 55.245) (width 0.254) (layer B.Cu) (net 21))
 (segment (start 115.697 39.497) (end 115.697 32.512) (width 0.254) (layer B.Cu) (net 4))
 (segment (start 128.901467 36.960533) (end 128.901467 39.620467) (width 0.254) (layer B.Cu) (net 4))
 (segment (start 128.901467 39.620467) (end 125.468934 43.053) (width 0.254) (layer B.Cu) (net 4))
 (segment (start 125.468934 43.053) (end 119.253 43.053) (width 0.254) (layer B.Cu) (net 4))
 (segment (start 130.937 34.925) (end 128.901467 36.960533) (width 0.254) (layer B.Cu) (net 4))
 (segment (start 119.253 43.053) (end 115.697 39.497) (width 0.254) (layer B.Cu) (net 4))
 (segment (start 131.2945 70.652) (end 130.6195 69.977) (width 0.254) (layer B.Cu) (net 27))
 (segment (start 131.311 70.652) (end 131.2945 70.652) (width 0.254) (layer B.Cu) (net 27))
 (segment (start 131.986 69.977) (end 131.311 70.652) (width 0.254) (layer B.Cu) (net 27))
 (segment (start 132.207 69.977) (end 131.986 69.977) (width 0.254) (layer B.Cu) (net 27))
 (segment (start 131.786 70.652) (end 131.311 70.652) (width 0.254) (layer B.Cu) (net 27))
 (segment (start 134.62 67.818) (end 131.786 70.652) (width 0.254) (layer B.Cu) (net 27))
 (segment (start 133.477 52.705) (end 134.62 53.848) (width 0.254) (layer B.Cu) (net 27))
 (segment (start 134.62 53.848) (end 134.62 67.818) (width 0.254) (layer B.Cu) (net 27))
 (segment (start 135.140701 71.822299) (end 132.310999 74.652001) (width 0.254) (layer B.Cu) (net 26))
 (segment (start 132.310999 74.652001) (end 131.311 75.652) (width 0.254) (layer B.Cu) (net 26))
 (segment (start 135.140701 53.581299) (end 135.140701 71.822299) (width 0.254) (layer B.Cu) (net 26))
 (segment (start 136.017 52.705) (end 135.140701 53.581299) (width 0.254) (layer B.Cu) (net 26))
 (segment (start 130.726357 88.920143) (end 131.311 89.504786) (width 0.254) (layer B.Cu) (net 24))
 (segment (start 131.311 89.504786) (end 131.311 89.702) (width 0.254) (layer B.Cu) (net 24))
 (segment (start 146.685 52.705) (end 147.28825 53.30825) (width 0.254) (layer B.Cu) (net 11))
 (segment (start 146.177 52.705) (end 146.685 52.705) (width 0.254) (layer B.Cu) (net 11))
 (segment (start 147.28825 53.30825) (end 147.28825 69.18325) (width 0.254) (layer B.Cu) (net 11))
 (segment (start 147.27975 69.18325) (end 145.811 70.652) (width 0.254) (layer B.Cu) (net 11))
 (segment (start 147.28825 69.18325) (end 147.27975 69.18325) (width 0.254) (layer B.Cu) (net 11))
 (segment (start 141.097 52.705) (end 139.446 54.356) (width 0.254) (layer B.Cu) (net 24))
 (segment (start 136.779 54.356) (end 135.594711 55.540289) (width 0.254) (layer B.Cu) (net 24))
 (segment (start 139.446 54.356) (end 136.779 54.356) (width 0.254) (layer B.Cu) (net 24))
 (segment (start 132.565 89.702) (end 131.311 89.702) (width 0.254) (layer B.Cu) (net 24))
 (segment (start 135.594711 86.672289) (end 132.565 89.702) (width 0.254) (layer B.Cu) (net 24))
 (segment (start 135.594711 55.540289) (end 135.594711 86.672289) (width 0.254) (layer B.Cu) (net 24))
 (segment (start 143.637 52.705) (end 141.53199 54.81001) (width 0.254) (layer B.Cu) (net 23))
 (segment (start 141.53199 54.81001) (end 136.967056 54.81001) (width 0.254) (layer B.Cu) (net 23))
 (segment (start 136.967056 54.81001) (end 136.048721 55.728345) (width 0.254) (layer B.Cu) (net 23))
 (segment (start 136.048721 86.860346) (end 132.842 90.067067) (width 0.254) (layer B.Cu) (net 23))
 (segment (start 136.048721 55.728345) (end 136.048721 86.860346) (width 0.254) (layer B.Cu) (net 23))
 (segment (start 132.842 93.171) (end 131.311 94.702) (width 0.254) (layer B.Cu) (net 23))
 (segment (start 132.842 90.067067) (end 132.842 93.171) (width 0.254) (layer B.Cu) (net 23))
 (segment (start 147.74226 87.77074) (end 145.811 89.702) (width 0.254) (layer B.Cu) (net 12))
 (segment (start 146.177 50.165) (end 147.74226 51.73026) (width 0.254) (layer B.Cu) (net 12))
 (segment (start 147.74226 51.73026) (end 147.74226 87.77074) (width 0.254) (layer B.Cu) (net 12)))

